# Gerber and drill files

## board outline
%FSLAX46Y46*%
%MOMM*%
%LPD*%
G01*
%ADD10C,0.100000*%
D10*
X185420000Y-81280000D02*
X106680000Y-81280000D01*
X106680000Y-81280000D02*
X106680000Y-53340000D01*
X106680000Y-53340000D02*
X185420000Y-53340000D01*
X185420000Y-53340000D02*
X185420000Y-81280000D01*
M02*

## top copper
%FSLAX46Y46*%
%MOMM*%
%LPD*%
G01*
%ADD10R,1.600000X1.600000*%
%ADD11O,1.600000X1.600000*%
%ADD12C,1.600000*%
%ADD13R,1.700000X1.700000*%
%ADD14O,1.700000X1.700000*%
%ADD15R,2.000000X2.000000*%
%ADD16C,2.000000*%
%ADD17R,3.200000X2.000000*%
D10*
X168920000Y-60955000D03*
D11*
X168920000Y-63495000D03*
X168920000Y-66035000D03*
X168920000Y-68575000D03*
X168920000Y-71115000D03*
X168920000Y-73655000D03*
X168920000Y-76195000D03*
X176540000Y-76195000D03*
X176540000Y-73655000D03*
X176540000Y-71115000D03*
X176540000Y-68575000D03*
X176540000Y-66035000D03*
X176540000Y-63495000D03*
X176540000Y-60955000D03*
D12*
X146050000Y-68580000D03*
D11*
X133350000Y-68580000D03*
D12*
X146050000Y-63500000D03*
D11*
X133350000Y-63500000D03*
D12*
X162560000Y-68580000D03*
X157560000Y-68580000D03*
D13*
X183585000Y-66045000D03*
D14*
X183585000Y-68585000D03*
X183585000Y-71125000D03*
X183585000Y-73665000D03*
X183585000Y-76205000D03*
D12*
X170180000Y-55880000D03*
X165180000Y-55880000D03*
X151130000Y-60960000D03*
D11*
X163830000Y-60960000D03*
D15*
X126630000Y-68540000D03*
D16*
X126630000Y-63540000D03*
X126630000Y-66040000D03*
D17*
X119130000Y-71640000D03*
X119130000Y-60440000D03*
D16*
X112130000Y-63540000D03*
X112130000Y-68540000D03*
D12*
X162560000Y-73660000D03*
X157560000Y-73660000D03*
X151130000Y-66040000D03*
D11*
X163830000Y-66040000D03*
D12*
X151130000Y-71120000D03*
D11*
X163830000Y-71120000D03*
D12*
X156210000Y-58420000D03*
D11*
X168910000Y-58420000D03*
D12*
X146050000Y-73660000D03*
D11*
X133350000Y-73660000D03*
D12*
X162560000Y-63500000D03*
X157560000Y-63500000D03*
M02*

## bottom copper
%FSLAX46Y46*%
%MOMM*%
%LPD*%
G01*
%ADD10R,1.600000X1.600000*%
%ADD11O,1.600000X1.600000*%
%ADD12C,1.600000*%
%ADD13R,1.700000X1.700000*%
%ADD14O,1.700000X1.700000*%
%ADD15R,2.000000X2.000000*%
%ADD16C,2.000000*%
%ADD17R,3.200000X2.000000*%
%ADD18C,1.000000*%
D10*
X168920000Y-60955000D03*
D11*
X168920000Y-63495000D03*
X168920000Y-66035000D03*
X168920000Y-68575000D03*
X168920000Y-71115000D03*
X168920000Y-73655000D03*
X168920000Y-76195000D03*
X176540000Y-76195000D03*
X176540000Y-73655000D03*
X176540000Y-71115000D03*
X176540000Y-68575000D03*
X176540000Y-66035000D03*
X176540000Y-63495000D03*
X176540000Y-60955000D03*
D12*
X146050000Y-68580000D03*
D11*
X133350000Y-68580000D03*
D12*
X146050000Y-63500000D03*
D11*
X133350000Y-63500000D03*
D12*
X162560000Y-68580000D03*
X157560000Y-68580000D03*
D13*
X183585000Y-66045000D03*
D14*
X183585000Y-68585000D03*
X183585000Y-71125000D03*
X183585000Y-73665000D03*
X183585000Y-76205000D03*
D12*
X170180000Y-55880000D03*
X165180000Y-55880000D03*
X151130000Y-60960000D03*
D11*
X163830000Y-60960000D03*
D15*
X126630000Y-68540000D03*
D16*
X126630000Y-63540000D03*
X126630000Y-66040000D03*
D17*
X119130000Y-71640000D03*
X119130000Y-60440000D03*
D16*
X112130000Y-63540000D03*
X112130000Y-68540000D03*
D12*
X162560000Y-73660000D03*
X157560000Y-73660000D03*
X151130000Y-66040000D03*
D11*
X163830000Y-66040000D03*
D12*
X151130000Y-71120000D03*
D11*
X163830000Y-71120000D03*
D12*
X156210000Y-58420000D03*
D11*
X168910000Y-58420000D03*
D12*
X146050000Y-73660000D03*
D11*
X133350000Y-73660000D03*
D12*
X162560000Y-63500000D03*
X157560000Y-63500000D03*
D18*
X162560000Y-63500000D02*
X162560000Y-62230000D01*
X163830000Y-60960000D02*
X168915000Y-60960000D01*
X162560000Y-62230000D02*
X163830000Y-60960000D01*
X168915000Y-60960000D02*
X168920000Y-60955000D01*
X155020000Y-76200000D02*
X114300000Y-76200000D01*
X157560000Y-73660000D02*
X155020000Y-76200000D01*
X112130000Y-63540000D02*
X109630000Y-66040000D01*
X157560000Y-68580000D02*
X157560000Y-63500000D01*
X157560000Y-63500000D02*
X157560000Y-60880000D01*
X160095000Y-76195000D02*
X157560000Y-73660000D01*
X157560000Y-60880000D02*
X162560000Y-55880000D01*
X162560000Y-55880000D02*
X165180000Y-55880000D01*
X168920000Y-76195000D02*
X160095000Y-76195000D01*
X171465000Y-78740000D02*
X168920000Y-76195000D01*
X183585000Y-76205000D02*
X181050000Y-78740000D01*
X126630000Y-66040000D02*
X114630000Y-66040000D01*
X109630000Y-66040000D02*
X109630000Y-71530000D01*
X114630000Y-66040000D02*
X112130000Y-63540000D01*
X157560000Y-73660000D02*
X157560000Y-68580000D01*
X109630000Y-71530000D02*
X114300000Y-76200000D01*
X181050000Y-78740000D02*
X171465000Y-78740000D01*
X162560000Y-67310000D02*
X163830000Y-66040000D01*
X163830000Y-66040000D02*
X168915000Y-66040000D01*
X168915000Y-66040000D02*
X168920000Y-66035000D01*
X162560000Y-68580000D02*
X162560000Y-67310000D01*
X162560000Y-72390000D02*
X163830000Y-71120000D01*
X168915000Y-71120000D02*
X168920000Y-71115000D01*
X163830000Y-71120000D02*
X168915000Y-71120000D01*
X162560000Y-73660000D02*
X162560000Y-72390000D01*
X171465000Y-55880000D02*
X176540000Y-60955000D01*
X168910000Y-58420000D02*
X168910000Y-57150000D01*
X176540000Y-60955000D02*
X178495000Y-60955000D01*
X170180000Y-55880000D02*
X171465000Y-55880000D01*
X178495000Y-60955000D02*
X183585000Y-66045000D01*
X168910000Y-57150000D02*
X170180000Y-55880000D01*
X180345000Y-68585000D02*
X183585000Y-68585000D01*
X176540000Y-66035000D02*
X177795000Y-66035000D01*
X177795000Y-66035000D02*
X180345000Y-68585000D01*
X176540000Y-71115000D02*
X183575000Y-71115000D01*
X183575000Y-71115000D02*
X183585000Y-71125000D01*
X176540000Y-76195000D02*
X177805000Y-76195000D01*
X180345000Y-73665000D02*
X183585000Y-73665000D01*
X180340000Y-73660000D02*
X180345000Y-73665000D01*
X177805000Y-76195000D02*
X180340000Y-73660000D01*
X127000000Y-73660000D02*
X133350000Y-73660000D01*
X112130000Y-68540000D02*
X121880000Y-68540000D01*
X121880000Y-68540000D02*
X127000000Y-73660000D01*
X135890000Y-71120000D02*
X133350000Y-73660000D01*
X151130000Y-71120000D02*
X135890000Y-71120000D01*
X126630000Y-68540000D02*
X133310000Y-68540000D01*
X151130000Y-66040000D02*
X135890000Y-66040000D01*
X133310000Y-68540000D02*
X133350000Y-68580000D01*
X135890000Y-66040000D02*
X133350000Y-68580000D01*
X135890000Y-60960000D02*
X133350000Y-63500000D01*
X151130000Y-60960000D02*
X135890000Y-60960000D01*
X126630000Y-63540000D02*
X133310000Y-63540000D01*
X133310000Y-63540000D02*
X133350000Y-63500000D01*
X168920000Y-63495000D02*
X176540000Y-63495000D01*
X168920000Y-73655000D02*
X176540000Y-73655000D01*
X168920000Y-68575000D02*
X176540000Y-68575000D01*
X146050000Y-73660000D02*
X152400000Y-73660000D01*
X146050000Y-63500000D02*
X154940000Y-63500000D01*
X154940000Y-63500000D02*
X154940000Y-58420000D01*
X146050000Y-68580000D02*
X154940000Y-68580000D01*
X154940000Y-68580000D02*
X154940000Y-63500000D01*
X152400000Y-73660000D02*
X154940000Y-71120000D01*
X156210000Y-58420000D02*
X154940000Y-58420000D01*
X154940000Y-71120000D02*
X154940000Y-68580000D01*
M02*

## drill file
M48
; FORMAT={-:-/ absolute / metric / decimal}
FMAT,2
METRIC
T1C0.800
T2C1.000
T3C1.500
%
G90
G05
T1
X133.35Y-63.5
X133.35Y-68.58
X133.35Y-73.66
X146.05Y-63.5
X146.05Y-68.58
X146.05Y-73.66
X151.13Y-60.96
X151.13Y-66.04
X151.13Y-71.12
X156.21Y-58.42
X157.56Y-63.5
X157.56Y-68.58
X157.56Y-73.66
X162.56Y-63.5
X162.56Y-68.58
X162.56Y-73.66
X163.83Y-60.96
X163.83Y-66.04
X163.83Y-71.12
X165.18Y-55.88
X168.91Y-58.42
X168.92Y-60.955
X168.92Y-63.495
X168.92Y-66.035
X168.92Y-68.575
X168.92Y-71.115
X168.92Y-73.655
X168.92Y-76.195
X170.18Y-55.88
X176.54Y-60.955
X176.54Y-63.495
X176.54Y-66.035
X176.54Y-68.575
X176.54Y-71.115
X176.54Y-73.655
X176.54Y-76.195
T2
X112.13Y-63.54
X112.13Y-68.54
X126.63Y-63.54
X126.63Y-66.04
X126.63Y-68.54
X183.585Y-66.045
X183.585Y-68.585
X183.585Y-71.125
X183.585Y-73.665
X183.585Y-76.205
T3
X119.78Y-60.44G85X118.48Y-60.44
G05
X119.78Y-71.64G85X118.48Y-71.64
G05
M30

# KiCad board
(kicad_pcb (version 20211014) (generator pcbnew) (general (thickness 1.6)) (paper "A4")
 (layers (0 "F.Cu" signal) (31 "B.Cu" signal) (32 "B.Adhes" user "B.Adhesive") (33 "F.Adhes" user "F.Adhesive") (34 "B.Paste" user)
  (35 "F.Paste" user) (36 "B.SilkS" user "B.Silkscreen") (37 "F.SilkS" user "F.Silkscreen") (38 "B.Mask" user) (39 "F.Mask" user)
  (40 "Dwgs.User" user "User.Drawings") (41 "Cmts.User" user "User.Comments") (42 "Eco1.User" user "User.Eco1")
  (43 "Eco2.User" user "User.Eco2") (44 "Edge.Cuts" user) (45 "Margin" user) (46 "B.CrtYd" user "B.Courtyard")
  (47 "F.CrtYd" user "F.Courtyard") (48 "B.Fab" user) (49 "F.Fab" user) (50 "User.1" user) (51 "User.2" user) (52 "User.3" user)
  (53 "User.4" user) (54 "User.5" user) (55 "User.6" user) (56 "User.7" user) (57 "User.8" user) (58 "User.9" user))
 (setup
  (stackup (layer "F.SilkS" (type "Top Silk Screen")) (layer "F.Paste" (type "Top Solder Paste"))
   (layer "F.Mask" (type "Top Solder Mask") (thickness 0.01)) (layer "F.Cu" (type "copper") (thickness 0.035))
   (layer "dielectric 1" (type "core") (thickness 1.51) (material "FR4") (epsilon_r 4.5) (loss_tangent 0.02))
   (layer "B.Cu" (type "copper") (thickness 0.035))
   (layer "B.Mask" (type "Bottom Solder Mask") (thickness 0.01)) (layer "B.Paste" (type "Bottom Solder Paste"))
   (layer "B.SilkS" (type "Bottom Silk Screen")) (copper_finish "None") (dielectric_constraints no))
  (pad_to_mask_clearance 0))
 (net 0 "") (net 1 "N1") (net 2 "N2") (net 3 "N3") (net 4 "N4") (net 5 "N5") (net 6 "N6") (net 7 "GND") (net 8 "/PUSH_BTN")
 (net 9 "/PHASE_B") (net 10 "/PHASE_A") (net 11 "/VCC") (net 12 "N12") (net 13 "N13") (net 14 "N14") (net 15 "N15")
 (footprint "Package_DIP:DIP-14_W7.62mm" (layer "F.Cu") (at 168.92 60.955)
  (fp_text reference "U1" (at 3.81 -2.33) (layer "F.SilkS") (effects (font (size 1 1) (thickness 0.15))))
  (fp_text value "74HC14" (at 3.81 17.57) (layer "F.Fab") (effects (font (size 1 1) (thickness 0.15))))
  (pad "1" thru_hole rect locked (at 0 0) (size 1.6 1.6) (drill 0.8) (layers *.Cu *.Mask) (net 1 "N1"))
  (pad "2" thru_hole oval locked (at 0 2.54) (size 1.6 1.6) (drill 0.8) (layers *.Cu *.Mask) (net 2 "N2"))
  (pad "3" thru_hole oval locked (at 0 5.08) (size 1.6 1.6) (drill 0.8) (layers *.Cu *.Mask) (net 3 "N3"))
  (pad "4" thru_hole oval locked (at 0 7.62) (size 1.6 1.6) (drill 0.8) (layers *.Cu *.Mask) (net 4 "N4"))
  (pad "5" thru_hole oval locked (at 0 10.16) (size 1.6 1.6) (drill 0.8) (layers *.Cu *.Mask) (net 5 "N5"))
  (pad "6" thru_hole oval locked (at 0 12.7) (size 1.6 1.6) (drill 0.8) (layers *.Cu *.Mask) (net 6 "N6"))
  (pad "7" thru_hole oval locked (at 0 15.24) (size 1.6 1.6) (drill 0.8) (layers *.Cu *.Mask) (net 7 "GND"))
  (pad "8" thru_hole oval locked (at 7.62 15.24) (size 1.6 1.6) (drill 0.8) (layers *.Cu *.Mask) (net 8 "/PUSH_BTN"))
  (pad "9" thru_hole oval locked (at 7.62 12.7) (size 1.6 1.6) (drill 0.8) (layers *.Cu *.Mask) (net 6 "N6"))
  (pad "10" thru_hole oval locked (at 7.62 10.16) (size 1.6 1.6) (drill 0.8) (layers *.Cu *.Mask) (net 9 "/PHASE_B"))
  (pad "11" thru_hole oval locked (at 7.62 7.62) (size 1.6 1.6) (drill 0.8) (layers *.Cu *.Mask) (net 4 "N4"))
  (pad "12" thru_hole oval locked (at 7.62 5.08) (size 1.6 1.6) (drill 0.8) (layers *.Cu *.Mask) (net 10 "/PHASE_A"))
  (pad "13" thru_hole oval locked (at 7.62 2.54) (size 1.6 1.6) (drill 0.8) (layers *.Cu *.Mask) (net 2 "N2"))
  (pad "14" thru_hole oval locked (at 7.62 0) (size 1.6 1.6) (drill 0.8) (layers *.Cu *.Mask) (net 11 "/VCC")))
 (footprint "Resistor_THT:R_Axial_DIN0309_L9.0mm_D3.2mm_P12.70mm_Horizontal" (layer "F.Cu") (at 146.05 68.58 180)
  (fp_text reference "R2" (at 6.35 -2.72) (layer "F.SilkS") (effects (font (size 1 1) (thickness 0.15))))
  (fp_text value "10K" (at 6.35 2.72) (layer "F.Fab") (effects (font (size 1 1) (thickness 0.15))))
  (pad "1" thru_hole circle locked (at 0 0 180) (size 1.6 1.6) (drill 0.8) (layers *.Cu *.Mask) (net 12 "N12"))
  (pad "2" thru_hole oval locked (at 12.7 0 180) (size 1.6 1.6) (drill 0.8) (layers *.Cu *.Mask) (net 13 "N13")))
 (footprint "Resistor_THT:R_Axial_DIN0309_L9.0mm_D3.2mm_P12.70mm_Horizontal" (layer "F.Cu") (at 146.05 63.5 180)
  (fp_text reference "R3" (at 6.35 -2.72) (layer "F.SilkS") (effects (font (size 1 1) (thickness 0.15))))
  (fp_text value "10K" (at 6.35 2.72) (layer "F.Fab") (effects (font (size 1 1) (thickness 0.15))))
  (pad "1" thru_hole circle locked (at 0 0 180) (size 1.6 1.6) (drill 0.8) (layers *.Cu *.Mask) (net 12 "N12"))
  (pad "2" thru_hole oval locked (at 12.7 0 180) (size 1.6 1.6) (drill 0.8) (layers *.Cu *.Mask) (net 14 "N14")))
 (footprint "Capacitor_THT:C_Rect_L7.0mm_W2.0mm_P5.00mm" (layer "F.Cu") (at 162.56 68.58 180)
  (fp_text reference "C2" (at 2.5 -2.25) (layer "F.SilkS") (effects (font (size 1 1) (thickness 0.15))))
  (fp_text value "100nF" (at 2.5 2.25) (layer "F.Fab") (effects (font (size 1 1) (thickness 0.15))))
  (pad "1" thru_hole circle locked (at 0 0 180) (size 1.6 1.6) (drill 0.8) (layers *.Cu *.Mask) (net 3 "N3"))
  (pad "2" thru_hole circle locked (at 5 0 180) (size 1.6 1.6) (drill 0.8) (layers *.Cu *.Mask) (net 7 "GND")))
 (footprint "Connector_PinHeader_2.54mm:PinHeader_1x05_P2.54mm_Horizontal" (layer "F.Cu") (at 183.585 66.045)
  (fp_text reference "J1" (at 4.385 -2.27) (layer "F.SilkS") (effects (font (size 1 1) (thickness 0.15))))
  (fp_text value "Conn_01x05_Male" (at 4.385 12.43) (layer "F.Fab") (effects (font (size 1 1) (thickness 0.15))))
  (pad "1" thru_hole rect locked (at 0 0) (size 1.7 1.7) (drill 1) (layers *.Cu *.Mask) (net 11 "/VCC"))
  (pad "2" thru_hole oval locked (at 0 2.54) (size 1.7 1.7) (drill 1) (layers *.Cu *.Mask) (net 10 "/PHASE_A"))
  (pad "3" thru_hole oval locked (at 0 5.08) (size 1.7 1.7) (drill 1) (layers *.Cu *.Mask) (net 9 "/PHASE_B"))
  (pad "4" thru_hole oval locked (at 0 7.62) (size 1.7 1.7) (drill 1) (layers *.Cu *.Mask) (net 8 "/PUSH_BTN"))
  (pad "5" thru_hole oval locked (at 0 10.16) (size 1.7 1.7) (drill 1) (layers *.Cu *.Mask) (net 7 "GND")))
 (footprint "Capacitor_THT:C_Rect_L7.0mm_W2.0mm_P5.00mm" (layer "F.Cu") (at 170.18 55.88 180)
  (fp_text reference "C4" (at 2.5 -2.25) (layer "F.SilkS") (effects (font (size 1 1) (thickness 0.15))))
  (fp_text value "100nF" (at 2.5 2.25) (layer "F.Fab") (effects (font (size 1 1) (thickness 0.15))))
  (pad "1" thru_hole circle locked (at 0 0 180) (size 1.6 1.6) (drill 0.8) (layers *.Cu *.Mask) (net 11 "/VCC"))
  (pad "2" thru_hole circle locked (at 5 0 180) (size 1.6 1.6) (drill 0.8) (layers *.Cu *.Mask) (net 7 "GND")))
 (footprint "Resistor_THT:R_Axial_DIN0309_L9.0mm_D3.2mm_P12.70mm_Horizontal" (layer "F.Cu") (at 151.13 60.96)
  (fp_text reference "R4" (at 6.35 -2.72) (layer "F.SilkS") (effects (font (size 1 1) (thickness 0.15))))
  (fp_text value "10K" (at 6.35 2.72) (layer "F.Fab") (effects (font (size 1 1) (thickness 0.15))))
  (pad "1" thru_hole circle locked (at 0 0) (size 1.6 1.6) (drill 0.8) (layers *.Cu *.Mask) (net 14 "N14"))
  (pad "2" thru_hole oval locked (at 12.7 0) (size 1.6 1.6) (drill 0.8) (layers *.Cu *.Mask) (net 1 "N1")))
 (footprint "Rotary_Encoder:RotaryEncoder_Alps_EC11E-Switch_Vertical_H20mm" (layer "F.Cu") (at 126.63 68.54 180)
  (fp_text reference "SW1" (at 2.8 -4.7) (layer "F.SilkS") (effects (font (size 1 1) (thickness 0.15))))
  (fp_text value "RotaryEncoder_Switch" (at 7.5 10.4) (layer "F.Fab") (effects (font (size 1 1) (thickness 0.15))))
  (pad "A" thru_hole rect locked (at 0 0 180) (size 2 2) (drill 1) (layers *.Cu *.Mask) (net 13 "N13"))
  (pad "B" thru_hole circle locked (at 0 5 180) (size 2 2) (drill 1) (layers *.Cu *.Mask) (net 14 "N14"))
  (pad "C" thru_hole circle locked (at 0 2.5 180) (size 2 2) (drill 1) (layers *.Cu *.Mask) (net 7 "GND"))
  (pad "MP" thru_hole rect locked (at 7.5 -3.1 180) (size 3.2 2) (drill oval 2.8 1.5) (layers *.Cu *.Mask))
  (pad "MP" thru_hole rect locked (at 7.5 8.1 180) (size 3.2 2) (drill oval 2.8 1.5) (layers *.Cu *.Mask))
  (pad "S1" thru_hole circle locked (at 14.5 5 180) (size 2 2) (drill 1) (layers *.Cu *.Mask) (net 7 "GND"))
  (pad "S2" thru_hole circle locked (at 14.5 0 180) (size 2 2) (drill 1) (layers *.Cu *.Mask) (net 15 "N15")))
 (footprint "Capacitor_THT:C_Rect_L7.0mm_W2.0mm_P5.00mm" (layer "F.Cu") (at 162.56 73.66 180)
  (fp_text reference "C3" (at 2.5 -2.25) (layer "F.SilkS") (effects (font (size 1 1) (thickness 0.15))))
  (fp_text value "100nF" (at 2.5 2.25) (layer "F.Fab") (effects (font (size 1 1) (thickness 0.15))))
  (pad "1" thru_hole circle locked (at 0 0 180) (size 1.6 1.6) (drill 0.8) (layers *.Cu *.Mask) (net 5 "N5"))
  (pad "2" thru_hole circle locked (at 5 0 180) (size 1.6 1.6) (drill 0.8) (layers *.Cu *.Mask) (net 7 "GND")))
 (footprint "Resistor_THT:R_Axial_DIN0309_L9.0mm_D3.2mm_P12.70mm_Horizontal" (layer "F.Cu") (at 151.13 66.04)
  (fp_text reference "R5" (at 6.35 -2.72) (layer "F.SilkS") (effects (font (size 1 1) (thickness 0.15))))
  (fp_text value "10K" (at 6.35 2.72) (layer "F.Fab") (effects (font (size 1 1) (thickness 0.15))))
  (pad "1" thru_hole circle locked (at 0 0) (size 1.6 1.6) (drill 0.8) (layers *.Cu *.Mask) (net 13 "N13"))
  (pad "2" thru_hole oval locked (at 12.7 0) (size 1.6 1.6) (drill 0.8) (layers *.Cu *.Mask) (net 3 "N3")))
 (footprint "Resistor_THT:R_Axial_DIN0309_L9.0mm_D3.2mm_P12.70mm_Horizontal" (layer "F.Cu") (at 151.13 71.12)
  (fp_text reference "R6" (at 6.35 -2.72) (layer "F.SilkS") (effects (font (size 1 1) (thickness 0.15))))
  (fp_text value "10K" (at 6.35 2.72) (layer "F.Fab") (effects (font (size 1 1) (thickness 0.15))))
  (pad "1" thru_hole circle locked (at 0 0) (size 1.6 1.6) (drill 0.8) (layers *.Cu *.Mask) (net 15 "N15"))
  (pad "2" thru_hole oval locked (at 12.7 0) (size 1.6 1.6) (drill 0.8) (layers *.Cu *.Mask) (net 5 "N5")))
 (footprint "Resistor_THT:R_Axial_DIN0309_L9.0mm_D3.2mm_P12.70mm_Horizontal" (layer "F.Cu") (at 156.21 58.42)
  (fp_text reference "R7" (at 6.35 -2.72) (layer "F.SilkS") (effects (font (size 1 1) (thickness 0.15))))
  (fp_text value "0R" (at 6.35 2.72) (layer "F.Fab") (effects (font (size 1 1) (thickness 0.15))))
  (pad "1" thru_hole circle locked (at 0 0) (size 1.6 1.6) (drill 0.8) (layers *.Cu *.Mask) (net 12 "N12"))
  (pad "2" thru_hole oval locked (at 12.7 0) (size 1.6 1.6) (drill 0.8) (layers *.Cu *.Mask) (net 11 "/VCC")))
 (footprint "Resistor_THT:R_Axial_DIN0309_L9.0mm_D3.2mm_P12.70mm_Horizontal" (layer "F.Cu") (at 146.05 73.66 180)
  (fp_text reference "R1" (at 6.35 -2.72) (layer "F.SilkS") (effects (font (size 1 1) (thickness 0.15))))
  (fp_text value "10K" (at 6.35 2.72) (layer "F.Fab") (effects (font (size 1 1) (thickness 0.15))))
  (pad "1" thru_hole circle locked (at 0 0 180) (size 1.6 1.6) (drill 0.8) (layers *.Cu *.Mask) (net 12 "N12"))
  (pad "2" thru_hole oval locked (at 12.7 0 180) (size 1.6 1.6) (drill 0.8) (layers *.Cu *.Mask) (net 15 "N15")))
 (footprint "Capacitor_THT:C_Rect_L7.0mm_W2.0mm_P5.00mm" (layer "F.Cu") (at 162.56 63.5 180)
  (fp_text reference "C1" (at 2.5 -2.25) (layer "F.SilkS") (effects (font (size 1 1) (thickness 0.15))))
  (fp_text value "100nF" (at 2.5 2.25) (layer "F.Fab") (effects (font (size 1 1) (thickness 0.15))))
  (pad "1" thru_hole circle locked (at 0 0 180) (size 1.6 1.6) (drill 0.8) (layers *.Cu *.Mask) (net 1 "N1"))
  (pad "2" thru_hole circle locked (at 5 0 180) (size 1.6 1.6) (drill 0.8) (layers *.Cu *.Mask) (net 7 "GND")))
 (gr_line (start 185.42 81.28) (end 106.68 81.28) (layer "Edge.Cuts") (width 0.1))
 (gr_line (start 106.68 81.28) (end 106.68 53.34) (layer "Edge.Cuts") (width 0.1))
 (gr_line (start 106.68 53.34) (end 185.42 53.34) (layer "Edge.Cuts") (width 0.1))
 (gr_line (start 185.42 53.34) (end 185.42 81.28) (layer "Edge.Cuts") (width 0.1))
 (segment (start 162.56 63.5) (end 162.56 62.23) (width 1) (layer "B.Cu") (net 1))
 (segment (start 163.83 60.96) (end 168.915 60.96) (width 1) (layer "B.Cu") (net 1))
 (segment (start 162.56 62.23) (end 163.83 60.96) (width 1) (layer "B.Cu") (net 1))
 (segment (start 168.915 60.96) (end 168.92 60.955) (width 1) (layer "B.Cu") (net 1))
 (segment (start 155.02 76.2) (end 114.3 76.2) (width 1) (layer "B.Cu") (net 7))
 (segment (start 157.56 73.66) (end 155.02 76.2) (width 1) (layer "B.Cu") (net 7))
 (segment (start 112.13 63.54) (end 109.63 66.04) (width 1) (layer "B.Cu") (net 7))
 (segment (start 157.56 68.58) (end 157.56 63.5) (width 1) (layer "B.Cu") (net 7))
 (segment (start 157.56 63.5) (end 157.56 60.88) (width 1) (layer "B.Cu") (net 7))
 (segment (start 160.095 76.195) (end 157.56 73.66) (width 1) (layer "B.Cu") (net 7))
 (segment (start 157.56 60.88) (end 162.56 55.88) (width 1) (layer "B.Cu") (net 7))
 (segment (start 162.56 55.88) (end 165.18 55.88) (width 1) (layer "B.Cu") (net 7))
 (segment (start 168.92 76.195) (end 160.095 76.195) (width 1) (layer "B.Cu") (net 7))
 (segment (start 171.465 78.74) (end 168.92 76.195) (width 1) (layer "B.Cu") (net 7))
 (segment (start 183.585 76.205) (end 181.05 78.74) (width 1) (layer "B.Cu") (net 7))
 (segment (start 126.63 66.04) (end 114.63 66.04) (width 1) (layer "B.Cu") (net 7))
 (segment (start 109.63 66.04) (end 109.63 71.53) (width 1) (layer "B.Cu") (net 7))
 (segment (start 114.63 66.04) (end 112.13 63.54) (width 1) (layer "B.Cu") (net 7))
 (segment (start 157.56 73.66) (end 157.56 68.58) (width 1) (layer "B.Cu") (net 7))
 (segment (start 109.63 71.53) (end 114.3 76.2) (width 1) (layer "B.Cu") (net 7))
 (segment (start 181.05 78.74) (end 171.465 78.74) (width 1) (layer "B.Cu") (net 7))
 (segment (start 162.56 67.31) (end 163.83 66.04) (width 1) (layer "B.Cu") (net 3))
 (segment (start 163.83 66.04) (end 168.915 66.04) (width 1) (layer "B.Cu") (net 3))
 (segment (start 168.915 66.04) (end 168.92 66.035) (width 1) (layer "B.Cu") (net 3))
 (segment (start 162.56 68.58) (end 162.56 67.31) (width 1) (layer "B.Cu") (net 3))
 (segment (start 162.56 72.39) (end 163.83 71.12) (width 1) (layer "B.Cu") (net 5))
 (segment (start 168.915 71.12) (end 168.92 71.115) (width 1) (layer "B.Cu") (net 5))
 (segment (start 163.83 71.12) (end 168.915 71.12) (width 1) (layer "B.Cu") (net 5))
 (segment (start 162.56 73.66) (end 162.56 72.39) (width 1) (layer "B.Cu") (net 5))
 (segment (start 171.465 55.88) (end 176.54 60.955) (width 1) (layer "B.Cu") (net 11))
 (segment (start 168.91 58.42) (end 168.91 57.15) (width 1) (layer "B.Cu") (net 11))
 (segment (start 176.54 60.955) (end 178.495 60.955) (width 1) (layer "B.Cu") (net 11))
 (segment (start 170.18 55.88) (end 171.465 55.88) (width 1) (layer "B.Cu") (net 11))
 (segment (start 178.495 60.955) (end 183.585 66.045) (width 1) (layer "B.Cu") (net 11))
 (segment (start 168.91 57.15) (end 170.18 55.88) (width 1) (layer "B.Cu") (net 11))
 (segment (start 180.345 68.585) (end 183.585 68.585) (width 1) (layer "B.Cu") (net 10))
 (segment (start 176.54 66.035) (end 177.795 66.035) (width 1) (layer "B.Cu") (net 10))
 (segment (start 177.795 66.035) (end 180.345 68.585) (width 1) (layer "B.Cu") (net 10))
 (segment (start 176.54 71.115) (end 183.575 71.115) (width 1) (layer "B.Cu") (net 9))
 (segment (start 183.575 71.115) (end 183.585 71.125) (width 1) (layer "B.Cu") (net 9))
 (segment (start 176.54 76.195) (end 177.805 76.195) (width 1) (layer "B.Cu") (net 8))
 (segment (start 180.345 73.665) (end 183.585 73.665) (width 1) (layer "B.Cu") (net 8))
 (segment (start 180.34 73.66) (end 180.345 73.665) (width 1) (layer "B.Cu") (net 8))
 (segment (start 177.805 76.195) (end 180.34 73.66) (width 1) (layer "B.Cu") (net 8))
 (segment (start 127 73.66) (end 133.35 73.66) (width 1) (layer "B.Cu") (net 15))
 (segment (start 112.13 68.54) (end 121.88 68.54) (width 1) (layer "B.Cu") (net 15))
 (segment (start 121.88 68.54) (end 127 73.66) (width 1) (layer "B.Cu") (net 15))
 (segment (start 135.89 71.12) (end 133.35 73.66) (width 1) (layer "B.Cu") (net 15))
 (segment (start 151.13 71.12) (end 135.89 71.12) (width 1) (layer "B.Cu") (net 15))
 (segment (start 126.63 68.54) (end 133.31 68.54) (width 1) (layer "B.Cu") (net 13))
 (segment (start 151.13 66.04) (end 135.89 66.04) (width 1) (layer "B.Cu") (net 13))
 (segment (start 133.31 68.54) (end 133.35 68.58) (width 1) (layer "B.Cu") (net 13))
 (segment (start 135.89 66.04) (end 133.35 68.58) (width 1) (layer "B.Cu") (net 13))
 (segment (start 135.89 60.96) (end 133.35 63.5) (width 1) (layer "B.Cu") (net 14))
 (segment (start 151.13 60.96) (end 135.89 60.96) (width 1) (layer "B.Cu") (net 14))
 (segment (start 126.63 63.54) (end 133.31 63.54) (width 1) (layer "B.Cu") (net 14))
 (segment (start 133.31 63.54) (end 133.35 63.5) (width 1) (layer "B.Cu") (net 14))
 (segment (start 168.92 63.495) (end 176.54 63.495) (width 1) (layer "B.Cu") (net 2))
 (segment (start 168.92 73.655) (end 176.54 73.655) (width 1) (layer "B.Cu") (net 6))
 (segment (start 168.92 68.575) (end 176.54 68.575) (width 1) (layer "B.Cu") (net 4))
 (segment (start 146.05 73.66) (end 152.4 73.66) (width 1) (layer "B.Cu") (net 12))
 (segment (start 146.05 63.5) (end 154.94 63.5) (width 1) (layer "B.Cu") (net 12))
 (segment (start 154.94 63.5) (end 154.94 58.42) (width 1) (layer "B.Cu") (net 12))
 (segment (start 146.05 68.58) (end 154.94 68.58) (width 1) (layer "B.Cu") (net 12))
 (segment (start 154.94 68.58) (end 154.94 63.5) (width 1) (layer "B.Cu") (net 12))
 (segment (start 152.4 73.66) (end 154.94 71.12) (width 1) (layer "B.Cu") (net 12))
 (segment (start 156.21 58.42) (end 154.94 58.42) (width 1) (layer "B.Cu") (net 12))
 (segment (start 154.94 71.12) (end 154.94 68.58) (width 1) (layer "B.Cu") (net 12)))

